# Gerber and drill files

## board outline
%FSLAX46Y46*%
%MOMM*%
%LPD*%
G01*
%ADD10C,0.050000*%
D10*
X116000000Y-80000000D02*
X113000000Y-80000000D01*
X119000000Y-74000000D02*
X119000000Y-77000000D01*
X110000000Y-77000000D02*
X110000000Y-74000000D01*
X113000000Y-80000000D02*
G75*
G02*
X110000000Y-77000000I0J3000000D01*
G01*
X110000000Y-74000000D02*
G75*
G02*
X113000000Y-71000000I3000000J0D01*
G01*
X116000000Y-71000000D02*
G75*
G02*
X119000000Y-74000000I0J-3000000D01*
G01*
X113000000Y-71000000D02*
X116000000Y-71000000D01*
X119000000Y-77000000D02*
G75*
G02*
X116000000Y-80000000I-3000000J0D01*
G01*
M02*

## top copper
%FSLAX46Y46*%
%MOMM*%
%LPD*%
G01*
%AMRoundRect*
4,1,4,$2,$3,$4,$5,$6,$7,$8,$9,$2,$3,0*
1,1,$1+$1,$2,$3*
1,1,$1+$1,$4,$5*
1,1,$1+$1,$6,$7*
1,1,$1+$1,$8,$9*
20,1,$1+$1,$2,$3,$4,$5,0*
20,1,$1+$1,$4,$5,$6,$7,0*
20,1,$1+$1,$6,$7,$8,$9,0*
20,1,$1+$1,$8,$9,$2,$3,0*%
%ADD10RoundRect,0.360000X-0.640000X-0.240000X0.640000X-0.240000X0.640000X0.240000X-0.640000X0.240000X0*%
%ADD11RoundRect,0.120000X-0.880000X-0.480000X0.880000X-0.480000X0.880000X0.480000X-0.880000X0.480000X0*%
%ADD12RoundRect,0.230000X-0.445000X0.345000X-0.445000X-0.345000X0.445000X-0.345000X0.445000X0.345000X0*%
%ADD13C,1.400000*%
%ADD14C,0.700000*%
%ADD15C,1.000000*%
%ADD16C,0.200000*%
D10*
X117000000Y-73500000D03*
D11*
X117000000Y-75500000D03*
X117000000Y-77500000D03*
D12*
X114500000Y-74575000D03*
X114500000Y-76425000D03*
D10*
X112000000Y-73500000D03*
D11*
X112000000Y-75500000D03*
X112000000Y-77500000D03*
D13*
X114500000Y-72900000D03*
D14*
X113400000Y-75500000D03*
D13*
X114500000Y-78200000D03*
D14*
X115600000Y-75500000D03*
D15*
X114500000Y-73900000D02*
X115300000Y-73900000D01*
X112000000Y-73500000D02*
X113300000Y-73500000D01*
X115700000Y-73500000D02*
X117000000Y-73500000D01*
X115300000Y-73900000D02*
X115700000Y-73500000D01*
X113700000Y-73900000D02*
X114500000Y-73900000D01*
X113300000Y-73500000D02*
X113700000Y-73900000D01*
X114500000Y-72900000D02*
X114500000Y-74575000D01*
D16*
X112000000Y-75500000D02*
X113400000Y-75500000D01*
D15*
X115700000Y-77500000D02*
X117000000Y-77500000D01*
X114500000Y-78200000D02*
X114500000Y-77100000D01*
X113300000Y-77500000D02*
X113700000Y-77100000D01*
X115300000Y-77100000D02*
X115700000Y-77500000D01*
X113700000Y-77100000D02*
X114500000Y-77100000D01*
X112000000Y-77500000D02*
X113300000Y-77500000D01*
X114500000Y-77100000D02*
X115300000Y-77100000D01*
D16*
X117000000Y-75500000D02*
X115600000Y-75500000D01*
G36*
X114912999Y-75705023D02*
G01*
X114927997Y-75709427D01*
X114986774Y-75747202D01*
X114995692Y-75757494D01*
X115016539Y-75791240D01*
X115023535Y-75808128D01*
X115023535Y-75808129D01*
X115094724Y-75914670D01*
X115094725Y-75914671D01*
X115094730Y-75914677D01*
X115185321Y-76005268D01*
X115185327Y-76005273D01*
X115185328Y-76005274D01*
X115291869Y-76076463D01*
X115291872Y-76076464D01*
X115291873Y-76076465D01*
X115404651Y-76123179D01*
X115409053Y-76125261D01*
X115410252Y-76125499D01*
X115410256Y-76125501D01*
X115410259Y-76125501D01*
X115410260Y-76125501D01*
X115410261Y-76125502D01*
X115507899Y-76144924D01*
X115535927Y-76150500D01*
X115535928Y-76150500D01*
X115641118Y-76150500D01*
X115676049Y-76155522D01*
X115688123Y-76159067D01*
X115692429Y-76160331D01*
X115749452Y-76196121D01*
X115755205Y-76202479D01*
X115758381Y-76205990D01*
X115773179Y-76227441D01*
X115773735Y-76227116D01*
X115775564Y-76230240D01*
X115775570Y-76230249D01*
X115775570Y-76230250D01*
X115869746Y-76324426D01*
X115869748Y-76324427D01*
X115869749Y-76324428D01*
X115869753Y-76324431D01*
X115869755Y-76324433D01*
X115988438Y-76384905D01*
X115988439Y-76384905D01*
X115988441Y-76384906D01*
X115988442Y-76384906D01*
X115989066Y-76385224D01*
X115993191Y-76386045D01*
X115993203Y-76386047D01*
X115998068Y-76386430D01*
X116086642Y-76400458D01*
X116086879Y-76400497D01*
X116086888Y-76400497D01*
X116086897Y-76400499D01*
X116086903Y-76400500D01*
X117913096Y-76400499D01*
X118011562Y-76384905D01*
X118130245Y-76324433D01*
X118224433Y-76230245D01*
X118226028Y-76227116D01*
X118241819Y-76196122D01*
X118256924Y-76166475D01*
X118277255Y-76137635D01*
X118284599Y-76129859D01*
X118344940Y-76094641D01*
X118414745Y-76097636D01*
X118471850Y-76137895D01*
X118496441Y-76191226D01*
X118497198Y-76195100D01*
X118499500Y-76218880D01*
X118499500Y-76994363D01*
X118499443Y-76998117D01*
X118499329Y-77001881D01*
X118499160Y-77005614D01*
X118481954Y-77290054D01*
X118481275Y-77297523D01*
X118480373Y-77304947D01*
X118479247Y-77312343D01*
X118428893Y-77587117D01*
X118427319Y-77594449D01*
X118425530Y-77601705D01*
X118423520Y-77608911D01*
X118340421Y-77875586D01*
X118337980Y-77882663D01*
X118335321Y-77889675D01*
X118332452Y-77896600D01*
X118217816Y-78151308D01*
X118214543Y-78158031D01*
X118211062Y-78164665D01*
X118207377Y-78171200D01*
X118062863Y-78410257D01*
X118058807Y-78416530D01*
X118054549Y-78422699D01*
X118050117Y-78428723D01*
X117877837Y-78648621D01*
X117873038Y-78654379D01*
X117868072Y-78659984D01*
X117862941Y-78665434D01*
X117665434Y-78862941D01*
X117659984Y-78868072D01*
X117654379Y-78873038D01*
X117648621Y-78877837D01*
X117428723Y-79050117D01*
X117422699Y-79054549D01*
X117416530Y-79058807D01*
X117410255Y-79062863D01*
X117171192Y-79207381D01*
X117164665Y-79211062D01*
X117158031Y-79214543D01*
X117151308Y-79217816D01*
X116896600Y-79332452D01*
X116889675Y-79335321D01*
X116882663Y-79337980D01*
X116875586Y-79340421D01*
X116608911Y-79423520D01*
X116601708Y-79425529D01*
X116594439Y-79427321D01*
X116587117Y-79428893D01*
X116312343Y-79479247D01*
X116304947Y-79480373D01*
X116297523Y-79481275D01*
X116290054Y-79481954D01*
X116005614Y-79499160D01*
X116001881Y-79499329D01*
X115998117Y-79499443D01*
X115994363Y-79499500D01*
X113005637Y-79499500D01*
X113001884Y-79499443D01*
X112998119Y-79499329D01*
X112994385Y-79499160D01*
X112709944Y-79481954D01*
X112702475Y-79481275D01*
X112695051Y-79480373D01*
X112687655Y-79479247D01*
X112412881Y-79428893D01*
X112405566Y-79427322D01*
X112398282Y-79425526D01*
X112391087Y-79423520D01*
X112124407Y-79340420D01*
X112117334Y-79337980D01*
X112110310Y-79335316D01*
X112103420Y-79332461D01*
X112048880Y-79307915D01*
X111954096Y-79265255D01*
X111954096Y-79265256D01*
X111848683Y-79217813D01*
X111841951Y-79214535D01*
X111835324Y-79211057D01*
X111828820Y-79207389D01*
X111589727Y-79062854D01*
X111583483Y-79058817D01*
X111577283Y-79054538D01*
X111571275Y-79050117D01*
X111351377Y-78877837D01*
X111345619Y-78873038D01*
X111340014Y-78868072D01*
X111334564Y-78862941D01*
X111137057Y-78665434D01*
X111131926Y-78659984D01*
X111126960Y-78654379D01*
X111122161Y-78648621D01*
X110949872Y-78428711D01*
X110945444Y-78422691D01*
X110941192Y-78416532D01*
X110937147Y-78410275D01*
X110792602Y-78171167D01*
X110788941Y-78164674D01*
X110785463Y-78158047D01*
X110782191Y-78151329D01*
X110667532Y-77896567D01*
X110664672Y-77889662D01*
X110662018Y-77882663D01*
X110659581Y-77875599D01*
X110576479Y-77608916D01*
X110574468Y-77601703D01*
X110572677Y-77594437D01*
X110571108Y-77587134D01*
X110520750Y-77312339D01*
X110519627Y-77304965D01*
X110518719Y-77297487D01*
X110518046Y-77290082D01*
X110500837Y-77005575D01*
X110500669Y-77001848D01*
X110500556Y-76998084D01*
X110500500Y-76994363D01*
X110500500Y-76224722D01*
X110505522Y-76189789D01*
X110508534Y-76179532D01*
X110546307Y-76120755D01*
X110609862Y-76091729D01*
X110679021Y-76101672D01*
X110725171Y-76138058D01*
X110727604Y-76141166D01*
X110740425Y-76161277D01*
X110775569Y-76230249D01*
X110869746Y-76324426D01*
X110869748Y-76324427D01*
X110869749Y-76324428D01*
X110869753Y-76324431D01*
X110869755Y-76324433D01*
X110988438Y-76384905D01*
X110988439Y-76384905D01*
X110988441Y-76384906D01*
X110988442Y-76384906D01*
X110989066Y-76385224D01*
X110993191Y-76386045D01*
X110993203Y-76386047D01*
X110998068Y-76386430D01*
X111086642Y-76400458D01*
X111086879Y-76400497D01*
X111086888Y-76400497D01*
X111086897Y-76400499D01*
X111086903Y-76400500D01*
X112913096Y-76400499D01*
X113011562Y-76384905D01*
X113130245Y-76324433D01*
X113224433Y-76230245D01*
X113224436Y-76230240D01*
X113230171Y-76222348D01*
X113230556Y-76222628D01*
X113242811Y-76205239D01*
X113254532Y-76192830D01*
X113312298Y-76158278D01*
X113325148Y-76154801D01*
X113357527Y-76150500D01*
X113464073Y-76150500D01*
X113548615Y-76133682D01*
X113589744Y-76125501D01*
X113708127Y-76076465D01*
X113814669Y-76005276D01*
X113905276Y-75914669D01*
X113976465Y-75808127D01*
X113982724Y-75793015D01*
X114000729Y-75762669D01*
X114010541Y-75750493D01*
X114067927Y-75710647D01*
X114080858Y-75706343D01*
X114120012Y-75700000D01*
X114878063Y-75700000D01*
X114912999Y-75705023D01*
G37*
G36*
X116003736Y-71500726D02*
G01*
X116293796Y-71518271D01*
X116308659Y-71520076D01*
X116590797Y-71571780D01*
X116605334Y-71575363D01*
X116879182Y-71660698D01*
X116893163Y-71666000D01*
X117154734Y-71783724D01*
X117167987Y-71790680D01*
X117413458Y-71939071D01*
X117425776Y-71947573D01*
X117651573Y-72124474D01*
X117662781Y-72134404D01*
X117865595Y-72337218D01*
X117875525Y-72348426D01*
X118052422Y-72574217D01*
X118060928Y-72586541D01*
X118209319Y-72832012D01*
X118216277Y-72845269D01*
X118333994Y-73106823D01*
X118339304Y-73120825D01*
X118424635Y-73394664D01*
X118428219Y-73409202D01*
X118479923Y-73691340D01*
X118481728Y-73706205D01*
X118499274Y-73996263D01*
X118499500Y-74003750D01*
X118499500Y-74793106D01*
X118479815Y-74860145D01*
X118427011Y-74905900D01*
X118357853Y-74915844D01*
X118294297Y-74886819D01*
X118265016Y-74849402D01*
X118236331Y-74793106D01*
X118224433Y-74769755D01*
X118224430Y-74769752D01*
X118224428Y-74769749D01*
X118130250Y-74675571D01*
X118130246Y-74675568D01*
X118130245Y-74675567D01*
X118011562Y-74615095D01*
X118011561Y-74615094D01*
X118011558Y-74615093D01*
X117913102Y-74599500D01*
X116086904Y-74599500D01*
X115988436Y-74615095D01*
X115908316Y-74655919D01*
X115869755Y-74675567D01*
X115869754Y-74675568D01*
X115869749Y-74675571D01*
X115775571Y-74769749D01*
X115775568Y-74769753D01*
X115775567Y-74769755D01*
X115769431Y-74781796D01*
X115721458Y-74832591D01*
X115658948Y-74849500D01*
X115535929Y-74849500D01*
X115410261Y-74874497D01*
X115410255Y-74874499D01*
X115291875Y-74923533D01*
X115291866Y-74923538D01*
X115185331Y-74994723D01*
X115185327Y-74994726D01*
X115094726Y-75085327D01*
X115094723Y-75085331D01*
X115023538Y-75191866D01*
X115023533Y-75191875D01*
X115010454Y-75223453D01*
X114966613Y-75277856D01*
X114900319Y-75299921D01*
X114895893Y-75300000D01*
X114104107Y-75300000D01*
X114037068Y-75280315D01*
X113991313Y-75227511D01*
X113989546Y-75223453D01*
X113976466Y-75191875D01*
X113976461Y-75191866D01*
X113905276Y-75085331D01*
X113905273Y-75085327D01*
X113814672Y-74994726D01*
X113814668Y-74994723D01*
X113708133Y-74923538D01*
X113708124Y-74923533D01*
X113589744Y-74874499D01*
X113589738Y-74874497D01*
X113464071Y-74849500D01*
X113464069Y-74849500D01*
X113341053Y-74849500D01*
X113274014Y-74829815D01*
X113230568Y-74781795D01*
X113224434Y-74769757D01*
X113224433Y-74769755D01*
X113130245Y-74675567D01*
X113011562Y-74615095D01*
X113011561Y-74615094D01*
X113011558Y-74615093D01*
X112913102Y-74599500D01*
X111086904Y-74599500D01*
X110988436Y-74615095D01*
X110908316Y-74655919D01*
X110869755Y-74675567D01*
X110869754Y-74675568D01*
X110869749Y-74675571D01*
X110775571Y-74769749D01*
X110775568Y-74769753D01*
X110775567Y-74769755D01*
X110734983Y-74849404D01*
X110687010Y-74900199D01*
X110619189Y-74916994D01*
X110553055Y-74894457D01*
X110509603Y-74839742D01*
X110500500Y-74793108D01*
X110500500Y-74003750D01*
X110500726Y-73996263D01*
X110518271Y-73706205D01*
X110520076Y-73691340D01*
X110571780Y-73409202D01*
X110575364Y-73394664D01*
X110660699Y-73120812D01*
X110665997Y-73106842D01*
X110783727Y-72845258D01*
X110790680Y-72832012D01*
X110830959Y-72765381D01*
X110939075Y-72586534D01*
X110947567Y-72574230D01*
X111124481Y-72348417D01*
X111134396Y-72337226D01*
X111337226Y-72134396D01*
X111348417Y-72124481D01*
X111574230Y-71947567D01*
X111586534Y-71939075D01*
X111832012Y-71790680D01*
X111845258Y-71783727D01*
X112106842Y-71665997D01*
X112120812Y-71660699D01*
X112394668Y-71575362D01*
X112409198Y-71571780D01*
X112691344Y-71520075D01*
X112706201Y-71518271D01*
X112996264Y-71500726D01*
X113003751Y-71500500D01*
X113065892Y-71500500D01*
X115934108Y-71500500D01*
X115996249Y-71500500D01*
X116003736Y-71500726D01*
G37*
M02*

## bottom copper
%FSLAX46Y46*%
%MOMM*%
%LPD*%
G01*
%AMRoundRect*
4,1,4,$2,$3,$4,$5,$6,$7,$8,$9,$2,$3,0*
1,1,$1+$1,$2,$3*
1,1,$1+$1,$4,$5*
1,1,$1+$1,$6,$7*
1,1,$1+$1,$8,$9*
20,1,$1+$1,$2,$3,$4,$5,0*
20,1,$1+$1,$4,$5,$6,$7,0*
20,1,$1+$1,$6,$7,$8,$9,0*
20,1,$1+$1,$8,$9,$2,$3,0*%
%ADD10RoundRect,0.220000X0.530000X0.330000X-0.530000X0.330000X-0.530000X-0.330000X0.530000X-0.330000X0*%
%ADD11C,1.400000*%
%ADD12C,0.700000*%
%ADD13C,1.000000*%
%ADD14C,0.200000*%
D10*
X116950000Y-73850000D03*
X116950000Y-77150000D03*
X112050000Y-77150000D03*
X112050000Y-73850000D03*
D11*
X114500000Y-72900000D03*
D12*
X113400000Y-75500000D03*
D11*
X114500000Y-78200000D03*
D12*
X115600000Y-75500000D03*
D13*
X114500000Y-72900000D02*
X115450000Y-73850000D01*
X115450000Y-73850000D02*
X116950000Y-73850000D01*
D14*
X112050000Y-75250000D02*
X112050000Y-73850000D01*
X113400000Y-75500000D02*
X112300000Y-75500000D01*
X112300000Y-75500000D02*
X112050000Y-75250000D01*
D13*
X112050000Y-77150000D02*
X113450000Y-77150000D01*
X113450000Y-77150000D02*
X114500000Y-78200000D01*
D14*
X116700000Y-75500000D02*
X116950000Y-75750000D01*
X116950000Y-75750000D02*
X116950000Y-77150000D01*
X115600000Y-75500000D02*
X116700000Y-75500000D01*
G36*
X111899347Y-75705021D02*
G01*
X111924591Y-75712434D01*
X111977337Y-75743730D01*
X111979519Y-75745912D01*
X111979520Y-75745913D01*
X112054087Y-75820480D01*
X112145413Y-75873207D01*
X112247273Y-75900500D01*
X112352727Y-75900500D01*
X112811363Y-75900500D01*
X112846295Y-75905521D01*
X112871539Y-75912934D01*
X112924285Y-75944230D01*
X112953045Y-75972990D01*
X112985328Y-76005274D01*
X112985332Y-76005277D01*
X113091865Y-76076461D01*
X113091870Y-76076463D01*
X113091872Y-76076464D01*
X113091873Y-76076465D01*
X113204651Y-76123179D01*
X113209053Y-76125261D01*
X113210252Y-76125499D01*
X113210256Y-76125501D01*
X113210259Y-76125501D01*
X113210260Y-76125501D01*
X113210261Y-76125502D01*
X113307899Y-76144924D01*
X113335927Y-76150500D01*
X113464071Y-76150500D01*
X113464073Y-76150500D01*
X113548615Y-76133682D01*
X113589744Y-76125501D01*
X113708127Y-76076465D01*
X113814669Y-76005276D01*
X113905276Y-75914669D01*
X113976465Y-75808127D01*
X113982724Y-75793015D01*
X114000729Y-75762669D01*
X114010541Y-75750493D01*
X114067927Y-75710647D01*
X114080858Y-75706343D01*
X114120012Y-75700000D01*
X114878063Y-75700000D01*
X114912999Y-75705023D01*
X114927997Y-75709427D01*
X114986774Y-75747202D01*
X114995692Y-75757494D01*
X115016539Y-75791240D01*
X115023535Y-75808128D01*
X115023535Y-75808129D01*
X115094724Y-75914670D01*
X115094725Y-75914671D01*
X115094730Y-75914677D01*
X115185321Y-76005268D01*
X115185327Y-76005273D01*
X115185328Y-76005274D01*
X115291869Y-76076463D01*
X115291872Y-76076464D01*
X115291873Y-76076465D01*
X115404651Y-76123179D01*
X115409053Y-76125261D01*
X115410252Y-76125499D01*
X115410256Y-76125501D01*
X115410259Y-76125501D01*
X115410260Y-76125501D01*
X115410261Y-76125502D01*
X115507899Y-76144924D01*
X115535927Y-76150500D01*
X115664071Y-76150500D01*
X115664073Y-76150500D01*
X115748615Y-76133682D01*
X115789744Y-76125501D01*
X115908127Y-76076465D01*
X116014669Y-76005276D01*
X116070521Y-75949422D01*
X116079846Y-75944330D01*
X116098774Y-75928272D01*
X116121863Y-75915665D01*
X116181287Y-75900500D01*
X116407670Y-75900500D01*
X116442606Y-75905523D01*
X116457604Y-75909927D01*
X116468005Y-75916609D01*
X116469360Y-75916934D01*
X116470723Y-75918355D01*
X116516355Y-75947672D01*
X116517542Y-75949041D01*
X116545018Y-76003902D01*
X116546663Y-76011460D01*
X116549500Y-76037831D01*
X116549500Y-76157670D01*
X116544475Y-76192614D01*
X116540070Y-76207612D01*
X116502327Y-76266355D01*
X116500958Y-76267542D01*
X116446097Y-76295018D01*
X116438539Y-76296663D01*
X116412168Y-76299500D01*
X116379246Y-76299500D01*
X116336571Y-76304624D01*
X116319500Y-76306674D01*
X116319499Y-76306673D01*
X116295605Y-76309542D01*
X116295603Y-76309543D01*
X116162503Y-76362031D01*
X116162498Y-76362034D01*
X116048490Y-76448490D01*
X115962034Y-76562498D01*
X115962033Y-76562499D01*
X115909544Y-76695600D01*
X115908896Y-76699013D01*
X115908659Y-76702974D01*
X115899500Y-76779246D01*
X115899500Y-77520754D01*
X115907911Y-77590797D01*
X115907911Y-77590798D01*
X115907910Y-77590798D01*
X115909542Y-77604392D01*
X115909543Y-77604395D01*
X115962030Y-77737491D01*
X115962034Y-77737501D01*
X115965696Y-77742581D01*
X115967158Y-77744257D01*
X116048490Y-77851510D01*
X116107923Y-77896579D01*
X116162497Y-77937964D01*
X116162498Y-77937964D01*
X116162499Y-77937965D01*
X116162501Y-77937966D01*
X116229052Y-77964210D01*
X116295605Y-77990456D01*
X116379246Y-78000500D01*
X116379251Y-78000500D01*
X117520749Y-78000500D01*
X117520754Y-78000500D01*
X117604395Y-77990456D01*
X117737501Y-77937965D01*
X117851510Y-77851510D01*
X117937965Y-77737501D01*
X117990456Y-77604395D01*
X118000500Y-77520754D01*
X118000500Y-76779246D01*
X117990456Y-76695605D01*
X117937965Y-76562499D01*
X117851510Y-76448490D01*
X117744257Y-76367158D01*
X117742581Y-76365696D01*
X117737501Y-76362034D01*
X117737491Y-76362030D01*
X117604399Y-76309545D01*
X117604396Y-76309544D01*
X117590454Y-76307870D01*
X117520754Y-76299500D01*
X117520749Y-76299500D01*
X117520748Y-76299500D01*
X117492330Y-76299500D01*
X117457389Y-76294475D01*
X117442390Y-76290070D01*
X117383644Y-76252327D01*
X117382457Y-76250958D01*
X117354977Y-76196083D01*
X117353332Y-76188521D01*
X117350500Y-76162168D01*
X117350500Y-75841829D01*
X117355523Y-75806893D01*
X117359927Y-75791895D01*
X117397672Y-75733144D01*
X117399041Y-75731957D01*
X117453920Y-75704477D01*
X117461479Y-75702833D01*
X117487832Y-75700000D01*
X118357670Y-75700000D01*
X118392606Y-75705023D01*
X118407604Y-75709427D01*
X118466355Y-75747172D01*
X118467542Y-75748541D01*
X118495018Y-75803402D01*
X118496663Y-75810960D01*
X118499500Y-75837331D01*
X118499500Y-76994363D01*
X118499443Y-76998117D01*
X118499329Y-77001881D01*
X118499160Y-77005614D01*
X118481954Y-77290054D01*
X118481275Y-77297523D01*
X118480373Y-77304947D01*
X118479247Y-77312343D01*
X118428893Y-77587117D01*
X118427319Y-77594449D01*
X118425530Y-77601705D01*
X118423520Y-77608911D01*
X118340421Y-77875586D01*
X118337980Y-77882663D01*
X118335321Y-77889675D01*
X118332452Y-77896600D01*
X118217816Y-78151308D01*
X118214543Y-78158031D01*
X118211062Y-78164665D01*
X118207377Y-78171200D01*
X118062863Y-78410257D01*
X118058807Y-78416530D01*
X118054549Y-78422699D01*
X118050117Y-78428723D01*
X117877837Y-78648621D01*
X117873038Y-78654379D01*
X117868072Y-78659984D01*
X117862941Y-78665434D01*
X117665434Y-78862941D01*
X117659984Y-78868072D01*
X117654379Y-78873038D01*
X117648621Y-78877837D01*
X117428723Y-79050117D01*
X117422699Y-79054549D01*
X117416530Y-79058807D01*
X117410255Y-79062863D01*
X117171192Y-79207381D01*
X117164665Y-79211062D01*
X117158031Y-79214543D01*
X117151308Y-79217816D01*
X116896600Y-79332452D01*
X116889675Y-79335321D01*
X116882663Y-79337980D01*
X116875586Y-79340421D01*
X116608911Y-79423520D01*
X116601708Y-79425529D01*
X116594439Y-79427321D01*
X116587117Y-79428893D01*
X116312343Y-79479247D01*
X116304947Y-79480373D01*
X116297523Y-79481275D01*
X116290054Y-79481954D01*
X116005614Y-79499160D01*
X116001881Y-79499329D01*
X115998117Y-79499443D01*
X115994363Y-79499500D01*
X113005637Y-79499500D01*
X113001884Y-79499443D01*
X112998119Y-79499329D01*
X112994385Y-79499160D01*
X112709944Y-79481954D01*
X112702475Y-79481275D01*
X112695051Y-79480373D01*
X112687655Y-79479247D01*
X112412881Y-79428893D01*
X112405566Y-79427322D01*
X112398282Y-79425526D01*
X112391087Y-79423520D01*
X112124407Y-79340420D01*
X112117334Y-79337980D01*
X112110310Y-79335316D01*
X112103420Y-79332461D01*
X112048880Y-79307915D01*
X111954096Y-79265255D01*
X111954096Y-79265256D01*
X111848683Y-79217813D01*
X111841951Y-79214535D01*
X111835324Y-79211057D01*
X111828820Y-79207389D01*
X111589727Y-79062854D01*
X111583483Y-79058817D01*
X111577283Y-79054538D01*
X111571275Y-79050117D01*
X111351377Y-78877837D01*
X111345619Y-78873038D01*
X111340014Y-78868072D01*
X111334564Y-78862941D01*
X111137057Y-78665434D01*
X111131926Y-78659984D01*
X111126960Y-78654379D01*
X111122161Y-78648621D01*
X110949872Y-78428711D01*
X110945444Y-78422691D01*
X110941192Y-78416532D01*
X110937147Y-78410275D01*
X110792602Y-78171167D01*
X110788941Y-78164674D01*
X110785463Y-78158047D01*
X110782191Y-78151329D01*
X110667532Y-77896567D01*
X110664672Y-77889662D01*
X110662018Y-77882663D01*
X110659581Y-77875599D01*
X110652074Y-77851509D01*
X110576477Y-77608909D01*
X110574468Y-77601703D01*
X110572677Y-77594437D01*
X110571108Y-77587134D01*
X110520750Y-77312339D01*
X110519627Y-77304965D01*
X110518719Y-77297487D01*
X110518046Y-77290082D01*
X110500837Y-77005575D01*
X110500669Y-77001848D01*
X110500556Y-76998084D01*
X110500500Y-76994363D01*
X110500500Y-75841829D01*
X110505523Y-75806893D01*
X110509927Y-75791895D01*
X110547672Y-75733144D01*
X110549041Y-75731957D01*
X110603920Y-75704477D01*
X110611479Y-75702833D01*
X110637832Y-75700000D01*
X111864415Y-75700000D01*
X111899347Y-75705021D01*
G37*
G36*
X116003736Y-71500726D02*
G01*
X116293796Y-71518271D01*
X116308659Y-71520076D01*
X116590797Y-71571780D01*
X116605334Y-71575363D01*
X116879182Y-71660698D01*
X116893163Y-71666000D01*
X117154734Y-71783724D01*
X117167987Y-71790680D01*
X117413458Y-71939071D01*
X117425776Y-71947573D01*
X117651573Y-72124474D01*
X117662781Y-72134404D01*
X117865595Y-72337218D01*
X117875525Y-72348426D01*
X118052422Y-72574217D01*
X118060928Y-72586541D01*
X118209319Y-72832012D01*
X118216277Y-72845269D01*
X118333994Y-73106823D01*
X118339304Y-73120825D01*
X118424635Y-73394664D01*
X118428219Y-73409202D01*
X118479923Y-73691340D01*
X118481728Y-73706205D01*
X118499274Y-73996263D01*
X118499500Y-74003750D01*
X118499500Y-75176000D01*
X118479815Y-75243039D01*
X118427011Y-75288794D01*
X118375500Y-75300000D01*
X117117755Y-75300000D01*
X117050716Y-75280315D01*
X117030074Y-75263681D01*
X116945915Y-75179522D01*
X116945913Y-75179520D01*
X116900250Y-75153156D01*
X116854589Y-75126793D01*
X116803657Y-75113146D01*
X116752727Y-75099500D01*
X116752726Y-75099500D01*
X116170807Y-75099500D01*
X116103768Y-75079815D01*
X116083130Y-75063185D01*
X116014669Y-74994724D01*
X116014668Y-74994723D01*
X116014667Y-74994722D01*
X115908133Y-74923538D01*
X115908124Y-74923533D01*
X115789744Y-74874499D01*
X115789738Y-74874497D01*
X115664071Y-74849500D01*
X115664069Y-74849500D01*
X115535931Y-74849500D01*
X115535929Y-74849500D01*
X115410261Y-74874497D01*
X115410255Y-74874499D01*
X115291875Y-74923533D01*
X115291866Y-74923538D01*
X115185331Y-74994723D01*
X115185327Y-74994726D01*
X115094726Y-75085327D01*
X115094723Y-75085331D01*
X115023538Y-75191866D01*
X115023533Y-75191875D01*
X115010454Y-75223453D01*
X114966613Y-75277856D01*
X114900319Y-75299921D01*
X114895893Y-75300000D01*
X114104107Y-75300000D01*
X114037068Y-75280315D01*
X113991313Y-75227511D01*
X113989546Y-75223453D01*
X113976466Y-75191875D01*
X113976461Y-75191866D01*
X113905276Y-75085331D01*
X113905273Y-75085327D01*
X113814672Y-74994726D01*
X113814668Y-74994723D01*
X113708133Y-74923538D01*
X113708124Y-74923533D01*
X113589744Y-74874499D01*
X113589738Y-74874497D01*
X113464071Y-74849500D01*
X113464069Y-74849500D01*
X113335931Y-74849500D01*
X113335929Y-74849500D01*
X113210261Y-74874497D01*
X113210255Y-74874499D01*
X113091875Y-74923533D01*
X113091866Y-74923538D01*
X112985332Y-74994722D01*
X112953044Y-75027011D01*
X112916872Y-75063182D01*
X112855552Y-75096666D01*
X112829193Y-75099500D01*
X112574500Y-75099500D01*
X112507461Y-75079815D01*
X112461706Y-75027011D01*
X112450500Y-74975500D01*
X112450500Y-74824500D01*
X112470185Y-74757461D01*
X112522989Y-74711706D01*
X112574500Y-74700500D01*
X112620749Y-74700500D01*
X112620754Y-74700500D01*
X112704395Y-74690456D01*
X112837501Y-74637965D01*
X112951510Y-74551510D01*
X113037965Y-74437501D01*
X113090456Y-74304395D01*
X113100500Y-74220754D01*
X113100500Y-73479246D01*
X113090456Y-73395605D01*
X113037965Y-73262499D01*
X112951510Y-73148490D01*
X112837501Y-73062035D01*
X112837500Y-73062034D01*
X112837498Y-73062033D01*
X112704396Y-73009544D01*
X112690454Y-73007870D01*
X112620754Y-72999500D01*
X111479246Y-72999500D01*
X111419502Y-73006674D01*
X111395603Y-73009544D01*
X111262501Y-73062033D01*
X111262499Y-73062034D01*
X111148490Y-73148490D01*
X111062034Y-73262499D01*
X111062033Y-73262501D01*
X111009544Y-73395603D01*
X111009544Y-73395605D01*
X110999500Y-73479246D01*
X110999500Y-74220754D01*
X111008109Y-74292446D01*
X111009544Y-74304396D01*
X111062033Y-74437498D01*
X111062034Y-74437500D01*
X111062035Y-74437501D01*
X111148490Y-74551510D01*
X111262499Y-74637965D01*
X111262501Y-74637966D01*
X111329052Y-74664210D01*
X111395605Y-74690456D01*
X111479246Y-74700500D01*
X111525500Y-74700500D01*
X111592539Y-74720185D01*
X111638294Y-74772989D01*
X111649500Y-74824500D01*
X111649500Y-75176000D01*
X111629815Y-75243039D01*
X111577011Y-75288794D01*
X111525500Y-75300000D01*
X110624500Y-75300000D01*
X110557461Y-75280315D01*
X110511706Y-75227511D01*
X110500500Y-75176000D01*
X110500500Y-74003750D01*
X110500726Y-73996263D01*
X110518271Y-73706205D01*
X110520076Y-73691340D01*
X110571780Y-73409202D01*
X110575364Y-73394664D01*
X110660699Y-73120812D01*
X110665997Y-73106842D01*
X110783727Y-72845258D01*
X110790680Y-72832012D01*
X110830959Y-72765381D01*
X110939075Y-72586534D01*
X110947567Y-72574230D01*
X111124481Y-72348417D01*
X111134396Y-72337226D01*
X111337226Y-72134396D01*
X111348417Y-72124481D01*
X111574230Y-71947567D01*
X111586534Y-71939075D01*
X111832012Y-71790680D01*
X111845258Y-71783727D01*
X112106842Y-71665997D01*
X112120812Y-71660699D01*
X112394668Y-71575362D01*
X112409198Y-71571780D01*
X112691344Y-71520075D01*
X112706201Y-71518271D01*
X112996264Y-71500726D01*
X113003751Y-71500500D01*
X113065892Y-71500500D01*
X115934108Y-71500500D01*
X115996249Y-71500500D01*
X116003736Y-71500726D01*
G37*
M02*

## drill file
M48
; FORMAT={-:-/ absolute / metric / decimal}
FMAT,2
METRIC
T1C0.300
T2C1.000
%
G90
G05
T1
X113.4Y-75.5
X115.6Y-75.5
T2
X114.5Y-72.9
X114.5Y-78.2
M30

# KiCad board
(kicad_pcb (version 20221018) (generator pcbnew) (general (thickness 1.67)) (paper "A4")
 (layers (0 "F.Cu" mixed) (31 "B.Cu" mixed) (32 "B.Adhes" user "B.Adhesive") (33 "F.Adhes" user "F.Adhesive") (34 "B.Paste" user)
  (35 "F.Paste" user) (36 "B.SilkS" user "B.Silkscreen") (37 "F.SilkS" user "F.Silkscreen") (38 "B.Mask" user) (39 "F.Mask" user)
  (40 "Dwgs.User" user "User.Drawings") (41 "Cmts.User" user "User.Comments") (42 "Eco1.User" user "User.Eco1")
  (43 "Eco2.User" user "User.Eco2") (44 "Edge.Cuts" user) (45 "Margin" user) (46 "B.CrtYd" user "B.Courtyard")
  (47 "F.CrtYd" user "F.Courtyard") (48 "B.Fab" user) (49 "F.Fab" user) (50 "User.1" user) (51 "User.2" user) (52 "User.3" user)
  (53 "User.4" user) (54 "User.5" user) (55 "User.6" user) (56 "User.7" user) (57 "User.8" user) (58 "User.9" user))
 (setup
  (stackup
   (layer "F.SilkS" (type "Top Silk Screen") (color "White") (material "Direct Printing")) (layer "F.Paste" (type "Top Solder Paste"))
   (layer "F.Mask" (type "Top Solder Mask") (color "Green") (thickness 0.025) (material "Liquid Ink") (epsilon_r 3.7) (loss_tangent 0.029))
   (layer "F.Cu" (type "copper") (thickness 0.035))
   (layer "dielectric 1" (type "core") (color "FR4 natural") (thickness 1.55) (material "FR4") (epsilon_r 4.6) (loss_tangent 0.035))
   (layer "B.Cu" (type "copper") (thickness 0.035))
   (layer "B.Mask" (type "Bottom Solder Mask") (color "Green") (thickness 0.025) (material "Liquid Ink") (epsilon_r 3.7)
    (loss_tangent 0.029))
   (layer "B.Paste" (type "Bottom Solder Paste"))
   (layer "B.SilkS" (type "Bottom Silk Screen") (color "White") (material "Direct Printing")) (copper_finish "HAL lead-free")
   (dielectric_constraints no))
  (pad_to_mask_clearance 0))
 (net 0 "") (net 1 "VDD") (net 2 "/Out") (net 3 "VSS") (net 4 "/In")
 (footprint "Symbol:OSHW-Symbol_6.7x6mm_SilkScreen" (layer "F.Cu") (at 138.7 87.6)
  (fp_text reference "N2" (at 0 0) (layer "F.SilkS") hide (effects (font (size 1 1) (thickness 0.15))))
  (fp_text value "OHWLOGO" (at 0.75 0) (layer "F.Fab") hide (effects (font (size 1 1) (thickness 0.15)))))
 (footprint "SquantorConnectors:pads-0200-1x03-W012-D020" (layer "F.Cu") (at 117 75.5)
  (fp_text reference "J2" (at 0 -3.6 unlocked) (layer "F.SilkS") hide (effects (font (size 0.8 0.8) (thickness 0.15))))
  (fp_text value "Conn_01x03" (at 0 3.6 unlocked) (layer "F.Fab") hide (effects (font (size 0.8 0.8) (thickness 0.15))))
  (pad "1" smd roundrect (at 0 -2) (size 2 1.2) (layers "F.Cu" "F.Paste" "F.Mask") (roundrect_rratio 0.3) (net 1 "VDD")
   (thermal_bridge_angle 45))
  (pad "2" smd roundrect (at 0 0) (size 2 1.2) (layers "F.Cu" "F.Paste" "F.Mask") (roundrect_rratio 0.1) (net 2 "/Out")
   (thermal_bridge_angle 45))
  (pad "3" smd roundrect (at 0 2) (size 2 1.2) (layers "F.Cu" "F.Paste" "F.Mask") (roundrect_rratio 0.1) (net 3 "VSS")
   (thermal_bridge_angle 45)))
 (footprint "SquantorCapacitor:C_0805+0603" (layer "F.Cu") (at 114.5 75.5 -90)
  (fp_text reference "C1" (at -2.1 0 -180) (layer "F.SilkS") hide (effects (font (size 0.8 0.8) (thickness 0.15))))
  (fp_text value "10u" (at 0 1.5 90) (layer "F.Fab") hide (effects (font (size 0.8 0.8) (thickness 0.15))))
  (pad "1" smd roundrect (at -0.925 0 270) (size 1.15 1.35) (layers "F.Cu" "F.Paste" "F.Mask") (roundrect_rratio 0.2) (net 1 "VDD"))
  (pad "2" smd roundrect (at 0.925 0 270) (size 1.15 1.35) (layers "F.Cu" "F.Paste" "F.Mask") (roundrect_rratio 0.2) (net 3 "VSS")))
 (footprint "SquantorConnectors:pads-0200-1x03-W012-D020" (layer "F.Cu") (at 112 75.5)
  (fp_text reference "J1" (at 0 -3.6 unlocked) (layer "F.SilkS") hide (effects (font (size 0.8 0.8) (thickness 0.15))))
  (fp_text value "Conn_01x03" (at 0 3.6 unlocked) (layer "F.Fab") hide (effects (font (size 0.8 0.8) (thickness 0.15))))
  (pad "1" smd roundrect (at 0 -2) (size 2 1.2) (layers "F.Cu" "F.Paste" "F.Mask") (roundrect_rratio 0.3) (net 1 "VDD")
   (thermal_bridge_angle 45))
  (pad "2" smd roundrect (at 0 0) (size 2 1.2) (layers "F.Cu" "F.Paste" "F.Mask") (roundrect_rratio 0.1) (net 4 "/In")
   (thermal_bridge_angle 45))
  (pad "3" smd roundrect (at 0 2) (size 2 1.2) (layers "F.Cu" "F.Paste" "F.Mask") (roundrect_rratio 0.1) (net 3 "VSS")
   (thermal_bridge_angle 45)))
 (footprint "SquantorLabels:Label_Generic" (layer "B.Cu") (at 114.5 78.8875 180)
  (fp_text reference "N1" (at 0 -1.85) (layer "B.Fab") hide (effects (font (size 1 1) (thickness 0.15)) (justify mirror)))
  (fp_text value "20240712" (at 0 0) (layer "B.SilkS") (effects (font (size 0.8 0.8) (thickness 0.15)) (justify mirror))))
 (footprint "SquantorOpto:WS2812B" (layer "B.Cu") (at 114.5 75.5 180)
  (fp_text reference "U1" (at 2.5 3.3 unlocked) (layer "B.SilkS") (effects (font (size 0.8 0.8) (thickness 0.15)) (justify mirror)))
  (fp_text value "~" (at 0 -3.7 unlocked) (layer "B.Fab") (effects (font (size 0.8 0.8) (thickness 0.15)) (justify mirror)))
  (pad "1" smd roundrect (at -2.45 1.65 180) (size 1.5 1.1) (layers "B.Cu" "B.Paste" "B.Mask") (roundrect_rratio 0.2) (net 1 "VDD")
   (thermal_bridge_angle 45))
  (pad "2" smd roundrect (at -2.45 -1.65 180) (size 1.5 1.1) (layers "B.Cu" "B.Paste" "B.Mask") (roundrect_rratio 0.2) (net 2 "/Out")
   (thermal_bridge_angle 45))
  (pad "3" smd roundrect (at 2.45 -1.65 180) (size 1.5 1.1) (layers "B.Cu" "B.Paste" "B.Mask") (roundrect_rratio 0.2) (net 3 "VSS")
   (thermal_bridge_angle 45))
  (pad "4" smd roundrect (at 2.45 1.65 180) (size 1.5 1.1) (layers "B.Cu" "B.Paste" "B.Mask") (roundrect_rratio 0.2) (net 4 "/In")
   (thermal_bridge_angle 45)))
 (gr_line (start 116 80) (end 113 80) (stroke (width 0.05) (type default)) (layer "Edge.Cuts"))
 (gr_line (start 119 74) (end 119 77) (stroke (width 0.05) (type default)) (layer "Edge.Cuts"))
 (gr_line (start 110 77) (end 110 74) (stroke (width 0.05) (type default)) (layer "Edge.Cuts"))
 (gr_arc (start 113 80) (mid 110.87868 79.12132) (end 110 77) (stroke (width 0.05) (type default)) (layer "Edge.Cuts"))
 (gr_arc (start 110 74) (mid 110.87868 71.87868) (end 113 71) (stroke (width 0.05) (type default)) (layer "Edge.Cuts"))
 (gr_arc (start 116 71) (mid 118.12132 71.87868) (end 119 74) (stroke (width 0.05) (type default)) (layer "Edge.Cuts"))
 (gr_line (start 113 71) (end 116 71) (stroke (width 0.05) (type default)) (layer "Edge.Cuts"))
 (gr_arc (start 119 77) (mid 118.12132 79.12132) (end 116 80) (stroke (width 0.05) (type default)) (layer "Edge.Cuts"))
 (segment (start 114.5 73.9) (end 115.3 73.9) (width 1) (layer "F.Cu") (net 1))
 (segment (start 112 73.5) (end 113.3 73.5) (width 1) (layer "F.Cu") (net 1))
 (segment (start 115.7 73.5) (end 117 73.5) (width 1) (layer "F.Cu") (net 1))
 (segment (start 115.3 73.9) (end 115.7 73.5) (width 1) (layer "F.Cu") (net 1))
 (segment (start 113.7 73.9) (end 114.5 73.9) (width 1) (layer "F.Cu") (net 1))
 (segment (start 113.3 73.5) (end 113.7 73.9) (width 1) (layer "F.Cu") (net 1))
 (segment (start 114.5 72.9) (end 114.5 74.575) (width 1) (layer "F.Cu") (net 1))
 (via (at 114.5 72.9) (size 1.4) (drill 1) (layers "F.Cu" "B.Cu") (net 1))
 (segment (start 114.5 72.9) (end 115.45 73.85) (width 1) (layer "B.Cu") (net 1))
 (segment (start 115.45 73.85) (end 116.95 73.85) (width 1) (layer "B.Cu") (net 1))
 (segment (start 112 75.5) (end 113.4 75.5) (width 0.2) (layer "F.Cu") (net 4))
 (via (at 113.4 75.5) (size 0.7) (drill 0.3) (layers "F.Cu" "B.Cu") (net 4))
 (segment (start 112.05 75.25) (end 112.05 73.85) (width 0.2) (layer "B.Cu") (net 4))
 (segment (start 113.4 75.5) (end 112.3 75.5) (width 0.2) (layer "B.Cu") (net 4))
 (segment (start 112.3 75.5) (end 112.05 75.25) (width 0.2) (layer "B.Cu") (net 4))
 (segment (start 115.7 77.5) (end 117 77.5) (width 1) (layer "F.Cu") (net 3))
 (segment (start 114.5 78.2) (end 114.5 77.1) (width 1) (layer "F.Cu") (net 3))
 (segment (start 113.3 77.5) (end 113.7 77.1) (width 1) (layer "F.Cu") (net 3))
 (segment (start 115.3 77.1) (end 115.7 77.5) (width 1) (layer "F.Cu") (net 3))
 (segment (start 113.7 77.1) (end 114.5 77.1) (width 1) (layer "F.Cu") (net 3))
 (segment (start 112 77.5) (end 113.3 77.5) (width 1) (layer "F.Cu") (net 3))
 (segment (start 114.5 77.1) (end 115.3 77.1) (width 1) (layer "F.Cu") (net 3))
 (via (at 114.5 78.2) (size 1.4) (drill 1) (layers "F.Cu" "B.Cu") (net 3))
 (segment (start 112.05 77.15) (end 113.45 77.15) (width 1) (layer "B.Cu") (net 3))
 (segment (start 113.45 77.15) (end 114.5 78.2) (width 1) (layer "B.Cu") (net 3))
 (segment (start 117 75.5) (end 115.6 75.5) (width 0.2) (layer "F.Cu") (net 2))
 (via (at 115.6 75.5) (size 0.7) (drill 0.3) (layers "F.Cu" "B.Cu") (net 2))
 (segment (start 116.7 75.5) (end 116.95 75.75) (width 0.2) (layer "B.Cu") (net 2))
 (segment (start 116.95 75.75) (end 116.95 77.15) (width 0.2) (layer "B.Cu") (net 2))
 (segment (start 115.6 75.5) (end 116.7 75.5) (width 0.2) (layer "B.Cu") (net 2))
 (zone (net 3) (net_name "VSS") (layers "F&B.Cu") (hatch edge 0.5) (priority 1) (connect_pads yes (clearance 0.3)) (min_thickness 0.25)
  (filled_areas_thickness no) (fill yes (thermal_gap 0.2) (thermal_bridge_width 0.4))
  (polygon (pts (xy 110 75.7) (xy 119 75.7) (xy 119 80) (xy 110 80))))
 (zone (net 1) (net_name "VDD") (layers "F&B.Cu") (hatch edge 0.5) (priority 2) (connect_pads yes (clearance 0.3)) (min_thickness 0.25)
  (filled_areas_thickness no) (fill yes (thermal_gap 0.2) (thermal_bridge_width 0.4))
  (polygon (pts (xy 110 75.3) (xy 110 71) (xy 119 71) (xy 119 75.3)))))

